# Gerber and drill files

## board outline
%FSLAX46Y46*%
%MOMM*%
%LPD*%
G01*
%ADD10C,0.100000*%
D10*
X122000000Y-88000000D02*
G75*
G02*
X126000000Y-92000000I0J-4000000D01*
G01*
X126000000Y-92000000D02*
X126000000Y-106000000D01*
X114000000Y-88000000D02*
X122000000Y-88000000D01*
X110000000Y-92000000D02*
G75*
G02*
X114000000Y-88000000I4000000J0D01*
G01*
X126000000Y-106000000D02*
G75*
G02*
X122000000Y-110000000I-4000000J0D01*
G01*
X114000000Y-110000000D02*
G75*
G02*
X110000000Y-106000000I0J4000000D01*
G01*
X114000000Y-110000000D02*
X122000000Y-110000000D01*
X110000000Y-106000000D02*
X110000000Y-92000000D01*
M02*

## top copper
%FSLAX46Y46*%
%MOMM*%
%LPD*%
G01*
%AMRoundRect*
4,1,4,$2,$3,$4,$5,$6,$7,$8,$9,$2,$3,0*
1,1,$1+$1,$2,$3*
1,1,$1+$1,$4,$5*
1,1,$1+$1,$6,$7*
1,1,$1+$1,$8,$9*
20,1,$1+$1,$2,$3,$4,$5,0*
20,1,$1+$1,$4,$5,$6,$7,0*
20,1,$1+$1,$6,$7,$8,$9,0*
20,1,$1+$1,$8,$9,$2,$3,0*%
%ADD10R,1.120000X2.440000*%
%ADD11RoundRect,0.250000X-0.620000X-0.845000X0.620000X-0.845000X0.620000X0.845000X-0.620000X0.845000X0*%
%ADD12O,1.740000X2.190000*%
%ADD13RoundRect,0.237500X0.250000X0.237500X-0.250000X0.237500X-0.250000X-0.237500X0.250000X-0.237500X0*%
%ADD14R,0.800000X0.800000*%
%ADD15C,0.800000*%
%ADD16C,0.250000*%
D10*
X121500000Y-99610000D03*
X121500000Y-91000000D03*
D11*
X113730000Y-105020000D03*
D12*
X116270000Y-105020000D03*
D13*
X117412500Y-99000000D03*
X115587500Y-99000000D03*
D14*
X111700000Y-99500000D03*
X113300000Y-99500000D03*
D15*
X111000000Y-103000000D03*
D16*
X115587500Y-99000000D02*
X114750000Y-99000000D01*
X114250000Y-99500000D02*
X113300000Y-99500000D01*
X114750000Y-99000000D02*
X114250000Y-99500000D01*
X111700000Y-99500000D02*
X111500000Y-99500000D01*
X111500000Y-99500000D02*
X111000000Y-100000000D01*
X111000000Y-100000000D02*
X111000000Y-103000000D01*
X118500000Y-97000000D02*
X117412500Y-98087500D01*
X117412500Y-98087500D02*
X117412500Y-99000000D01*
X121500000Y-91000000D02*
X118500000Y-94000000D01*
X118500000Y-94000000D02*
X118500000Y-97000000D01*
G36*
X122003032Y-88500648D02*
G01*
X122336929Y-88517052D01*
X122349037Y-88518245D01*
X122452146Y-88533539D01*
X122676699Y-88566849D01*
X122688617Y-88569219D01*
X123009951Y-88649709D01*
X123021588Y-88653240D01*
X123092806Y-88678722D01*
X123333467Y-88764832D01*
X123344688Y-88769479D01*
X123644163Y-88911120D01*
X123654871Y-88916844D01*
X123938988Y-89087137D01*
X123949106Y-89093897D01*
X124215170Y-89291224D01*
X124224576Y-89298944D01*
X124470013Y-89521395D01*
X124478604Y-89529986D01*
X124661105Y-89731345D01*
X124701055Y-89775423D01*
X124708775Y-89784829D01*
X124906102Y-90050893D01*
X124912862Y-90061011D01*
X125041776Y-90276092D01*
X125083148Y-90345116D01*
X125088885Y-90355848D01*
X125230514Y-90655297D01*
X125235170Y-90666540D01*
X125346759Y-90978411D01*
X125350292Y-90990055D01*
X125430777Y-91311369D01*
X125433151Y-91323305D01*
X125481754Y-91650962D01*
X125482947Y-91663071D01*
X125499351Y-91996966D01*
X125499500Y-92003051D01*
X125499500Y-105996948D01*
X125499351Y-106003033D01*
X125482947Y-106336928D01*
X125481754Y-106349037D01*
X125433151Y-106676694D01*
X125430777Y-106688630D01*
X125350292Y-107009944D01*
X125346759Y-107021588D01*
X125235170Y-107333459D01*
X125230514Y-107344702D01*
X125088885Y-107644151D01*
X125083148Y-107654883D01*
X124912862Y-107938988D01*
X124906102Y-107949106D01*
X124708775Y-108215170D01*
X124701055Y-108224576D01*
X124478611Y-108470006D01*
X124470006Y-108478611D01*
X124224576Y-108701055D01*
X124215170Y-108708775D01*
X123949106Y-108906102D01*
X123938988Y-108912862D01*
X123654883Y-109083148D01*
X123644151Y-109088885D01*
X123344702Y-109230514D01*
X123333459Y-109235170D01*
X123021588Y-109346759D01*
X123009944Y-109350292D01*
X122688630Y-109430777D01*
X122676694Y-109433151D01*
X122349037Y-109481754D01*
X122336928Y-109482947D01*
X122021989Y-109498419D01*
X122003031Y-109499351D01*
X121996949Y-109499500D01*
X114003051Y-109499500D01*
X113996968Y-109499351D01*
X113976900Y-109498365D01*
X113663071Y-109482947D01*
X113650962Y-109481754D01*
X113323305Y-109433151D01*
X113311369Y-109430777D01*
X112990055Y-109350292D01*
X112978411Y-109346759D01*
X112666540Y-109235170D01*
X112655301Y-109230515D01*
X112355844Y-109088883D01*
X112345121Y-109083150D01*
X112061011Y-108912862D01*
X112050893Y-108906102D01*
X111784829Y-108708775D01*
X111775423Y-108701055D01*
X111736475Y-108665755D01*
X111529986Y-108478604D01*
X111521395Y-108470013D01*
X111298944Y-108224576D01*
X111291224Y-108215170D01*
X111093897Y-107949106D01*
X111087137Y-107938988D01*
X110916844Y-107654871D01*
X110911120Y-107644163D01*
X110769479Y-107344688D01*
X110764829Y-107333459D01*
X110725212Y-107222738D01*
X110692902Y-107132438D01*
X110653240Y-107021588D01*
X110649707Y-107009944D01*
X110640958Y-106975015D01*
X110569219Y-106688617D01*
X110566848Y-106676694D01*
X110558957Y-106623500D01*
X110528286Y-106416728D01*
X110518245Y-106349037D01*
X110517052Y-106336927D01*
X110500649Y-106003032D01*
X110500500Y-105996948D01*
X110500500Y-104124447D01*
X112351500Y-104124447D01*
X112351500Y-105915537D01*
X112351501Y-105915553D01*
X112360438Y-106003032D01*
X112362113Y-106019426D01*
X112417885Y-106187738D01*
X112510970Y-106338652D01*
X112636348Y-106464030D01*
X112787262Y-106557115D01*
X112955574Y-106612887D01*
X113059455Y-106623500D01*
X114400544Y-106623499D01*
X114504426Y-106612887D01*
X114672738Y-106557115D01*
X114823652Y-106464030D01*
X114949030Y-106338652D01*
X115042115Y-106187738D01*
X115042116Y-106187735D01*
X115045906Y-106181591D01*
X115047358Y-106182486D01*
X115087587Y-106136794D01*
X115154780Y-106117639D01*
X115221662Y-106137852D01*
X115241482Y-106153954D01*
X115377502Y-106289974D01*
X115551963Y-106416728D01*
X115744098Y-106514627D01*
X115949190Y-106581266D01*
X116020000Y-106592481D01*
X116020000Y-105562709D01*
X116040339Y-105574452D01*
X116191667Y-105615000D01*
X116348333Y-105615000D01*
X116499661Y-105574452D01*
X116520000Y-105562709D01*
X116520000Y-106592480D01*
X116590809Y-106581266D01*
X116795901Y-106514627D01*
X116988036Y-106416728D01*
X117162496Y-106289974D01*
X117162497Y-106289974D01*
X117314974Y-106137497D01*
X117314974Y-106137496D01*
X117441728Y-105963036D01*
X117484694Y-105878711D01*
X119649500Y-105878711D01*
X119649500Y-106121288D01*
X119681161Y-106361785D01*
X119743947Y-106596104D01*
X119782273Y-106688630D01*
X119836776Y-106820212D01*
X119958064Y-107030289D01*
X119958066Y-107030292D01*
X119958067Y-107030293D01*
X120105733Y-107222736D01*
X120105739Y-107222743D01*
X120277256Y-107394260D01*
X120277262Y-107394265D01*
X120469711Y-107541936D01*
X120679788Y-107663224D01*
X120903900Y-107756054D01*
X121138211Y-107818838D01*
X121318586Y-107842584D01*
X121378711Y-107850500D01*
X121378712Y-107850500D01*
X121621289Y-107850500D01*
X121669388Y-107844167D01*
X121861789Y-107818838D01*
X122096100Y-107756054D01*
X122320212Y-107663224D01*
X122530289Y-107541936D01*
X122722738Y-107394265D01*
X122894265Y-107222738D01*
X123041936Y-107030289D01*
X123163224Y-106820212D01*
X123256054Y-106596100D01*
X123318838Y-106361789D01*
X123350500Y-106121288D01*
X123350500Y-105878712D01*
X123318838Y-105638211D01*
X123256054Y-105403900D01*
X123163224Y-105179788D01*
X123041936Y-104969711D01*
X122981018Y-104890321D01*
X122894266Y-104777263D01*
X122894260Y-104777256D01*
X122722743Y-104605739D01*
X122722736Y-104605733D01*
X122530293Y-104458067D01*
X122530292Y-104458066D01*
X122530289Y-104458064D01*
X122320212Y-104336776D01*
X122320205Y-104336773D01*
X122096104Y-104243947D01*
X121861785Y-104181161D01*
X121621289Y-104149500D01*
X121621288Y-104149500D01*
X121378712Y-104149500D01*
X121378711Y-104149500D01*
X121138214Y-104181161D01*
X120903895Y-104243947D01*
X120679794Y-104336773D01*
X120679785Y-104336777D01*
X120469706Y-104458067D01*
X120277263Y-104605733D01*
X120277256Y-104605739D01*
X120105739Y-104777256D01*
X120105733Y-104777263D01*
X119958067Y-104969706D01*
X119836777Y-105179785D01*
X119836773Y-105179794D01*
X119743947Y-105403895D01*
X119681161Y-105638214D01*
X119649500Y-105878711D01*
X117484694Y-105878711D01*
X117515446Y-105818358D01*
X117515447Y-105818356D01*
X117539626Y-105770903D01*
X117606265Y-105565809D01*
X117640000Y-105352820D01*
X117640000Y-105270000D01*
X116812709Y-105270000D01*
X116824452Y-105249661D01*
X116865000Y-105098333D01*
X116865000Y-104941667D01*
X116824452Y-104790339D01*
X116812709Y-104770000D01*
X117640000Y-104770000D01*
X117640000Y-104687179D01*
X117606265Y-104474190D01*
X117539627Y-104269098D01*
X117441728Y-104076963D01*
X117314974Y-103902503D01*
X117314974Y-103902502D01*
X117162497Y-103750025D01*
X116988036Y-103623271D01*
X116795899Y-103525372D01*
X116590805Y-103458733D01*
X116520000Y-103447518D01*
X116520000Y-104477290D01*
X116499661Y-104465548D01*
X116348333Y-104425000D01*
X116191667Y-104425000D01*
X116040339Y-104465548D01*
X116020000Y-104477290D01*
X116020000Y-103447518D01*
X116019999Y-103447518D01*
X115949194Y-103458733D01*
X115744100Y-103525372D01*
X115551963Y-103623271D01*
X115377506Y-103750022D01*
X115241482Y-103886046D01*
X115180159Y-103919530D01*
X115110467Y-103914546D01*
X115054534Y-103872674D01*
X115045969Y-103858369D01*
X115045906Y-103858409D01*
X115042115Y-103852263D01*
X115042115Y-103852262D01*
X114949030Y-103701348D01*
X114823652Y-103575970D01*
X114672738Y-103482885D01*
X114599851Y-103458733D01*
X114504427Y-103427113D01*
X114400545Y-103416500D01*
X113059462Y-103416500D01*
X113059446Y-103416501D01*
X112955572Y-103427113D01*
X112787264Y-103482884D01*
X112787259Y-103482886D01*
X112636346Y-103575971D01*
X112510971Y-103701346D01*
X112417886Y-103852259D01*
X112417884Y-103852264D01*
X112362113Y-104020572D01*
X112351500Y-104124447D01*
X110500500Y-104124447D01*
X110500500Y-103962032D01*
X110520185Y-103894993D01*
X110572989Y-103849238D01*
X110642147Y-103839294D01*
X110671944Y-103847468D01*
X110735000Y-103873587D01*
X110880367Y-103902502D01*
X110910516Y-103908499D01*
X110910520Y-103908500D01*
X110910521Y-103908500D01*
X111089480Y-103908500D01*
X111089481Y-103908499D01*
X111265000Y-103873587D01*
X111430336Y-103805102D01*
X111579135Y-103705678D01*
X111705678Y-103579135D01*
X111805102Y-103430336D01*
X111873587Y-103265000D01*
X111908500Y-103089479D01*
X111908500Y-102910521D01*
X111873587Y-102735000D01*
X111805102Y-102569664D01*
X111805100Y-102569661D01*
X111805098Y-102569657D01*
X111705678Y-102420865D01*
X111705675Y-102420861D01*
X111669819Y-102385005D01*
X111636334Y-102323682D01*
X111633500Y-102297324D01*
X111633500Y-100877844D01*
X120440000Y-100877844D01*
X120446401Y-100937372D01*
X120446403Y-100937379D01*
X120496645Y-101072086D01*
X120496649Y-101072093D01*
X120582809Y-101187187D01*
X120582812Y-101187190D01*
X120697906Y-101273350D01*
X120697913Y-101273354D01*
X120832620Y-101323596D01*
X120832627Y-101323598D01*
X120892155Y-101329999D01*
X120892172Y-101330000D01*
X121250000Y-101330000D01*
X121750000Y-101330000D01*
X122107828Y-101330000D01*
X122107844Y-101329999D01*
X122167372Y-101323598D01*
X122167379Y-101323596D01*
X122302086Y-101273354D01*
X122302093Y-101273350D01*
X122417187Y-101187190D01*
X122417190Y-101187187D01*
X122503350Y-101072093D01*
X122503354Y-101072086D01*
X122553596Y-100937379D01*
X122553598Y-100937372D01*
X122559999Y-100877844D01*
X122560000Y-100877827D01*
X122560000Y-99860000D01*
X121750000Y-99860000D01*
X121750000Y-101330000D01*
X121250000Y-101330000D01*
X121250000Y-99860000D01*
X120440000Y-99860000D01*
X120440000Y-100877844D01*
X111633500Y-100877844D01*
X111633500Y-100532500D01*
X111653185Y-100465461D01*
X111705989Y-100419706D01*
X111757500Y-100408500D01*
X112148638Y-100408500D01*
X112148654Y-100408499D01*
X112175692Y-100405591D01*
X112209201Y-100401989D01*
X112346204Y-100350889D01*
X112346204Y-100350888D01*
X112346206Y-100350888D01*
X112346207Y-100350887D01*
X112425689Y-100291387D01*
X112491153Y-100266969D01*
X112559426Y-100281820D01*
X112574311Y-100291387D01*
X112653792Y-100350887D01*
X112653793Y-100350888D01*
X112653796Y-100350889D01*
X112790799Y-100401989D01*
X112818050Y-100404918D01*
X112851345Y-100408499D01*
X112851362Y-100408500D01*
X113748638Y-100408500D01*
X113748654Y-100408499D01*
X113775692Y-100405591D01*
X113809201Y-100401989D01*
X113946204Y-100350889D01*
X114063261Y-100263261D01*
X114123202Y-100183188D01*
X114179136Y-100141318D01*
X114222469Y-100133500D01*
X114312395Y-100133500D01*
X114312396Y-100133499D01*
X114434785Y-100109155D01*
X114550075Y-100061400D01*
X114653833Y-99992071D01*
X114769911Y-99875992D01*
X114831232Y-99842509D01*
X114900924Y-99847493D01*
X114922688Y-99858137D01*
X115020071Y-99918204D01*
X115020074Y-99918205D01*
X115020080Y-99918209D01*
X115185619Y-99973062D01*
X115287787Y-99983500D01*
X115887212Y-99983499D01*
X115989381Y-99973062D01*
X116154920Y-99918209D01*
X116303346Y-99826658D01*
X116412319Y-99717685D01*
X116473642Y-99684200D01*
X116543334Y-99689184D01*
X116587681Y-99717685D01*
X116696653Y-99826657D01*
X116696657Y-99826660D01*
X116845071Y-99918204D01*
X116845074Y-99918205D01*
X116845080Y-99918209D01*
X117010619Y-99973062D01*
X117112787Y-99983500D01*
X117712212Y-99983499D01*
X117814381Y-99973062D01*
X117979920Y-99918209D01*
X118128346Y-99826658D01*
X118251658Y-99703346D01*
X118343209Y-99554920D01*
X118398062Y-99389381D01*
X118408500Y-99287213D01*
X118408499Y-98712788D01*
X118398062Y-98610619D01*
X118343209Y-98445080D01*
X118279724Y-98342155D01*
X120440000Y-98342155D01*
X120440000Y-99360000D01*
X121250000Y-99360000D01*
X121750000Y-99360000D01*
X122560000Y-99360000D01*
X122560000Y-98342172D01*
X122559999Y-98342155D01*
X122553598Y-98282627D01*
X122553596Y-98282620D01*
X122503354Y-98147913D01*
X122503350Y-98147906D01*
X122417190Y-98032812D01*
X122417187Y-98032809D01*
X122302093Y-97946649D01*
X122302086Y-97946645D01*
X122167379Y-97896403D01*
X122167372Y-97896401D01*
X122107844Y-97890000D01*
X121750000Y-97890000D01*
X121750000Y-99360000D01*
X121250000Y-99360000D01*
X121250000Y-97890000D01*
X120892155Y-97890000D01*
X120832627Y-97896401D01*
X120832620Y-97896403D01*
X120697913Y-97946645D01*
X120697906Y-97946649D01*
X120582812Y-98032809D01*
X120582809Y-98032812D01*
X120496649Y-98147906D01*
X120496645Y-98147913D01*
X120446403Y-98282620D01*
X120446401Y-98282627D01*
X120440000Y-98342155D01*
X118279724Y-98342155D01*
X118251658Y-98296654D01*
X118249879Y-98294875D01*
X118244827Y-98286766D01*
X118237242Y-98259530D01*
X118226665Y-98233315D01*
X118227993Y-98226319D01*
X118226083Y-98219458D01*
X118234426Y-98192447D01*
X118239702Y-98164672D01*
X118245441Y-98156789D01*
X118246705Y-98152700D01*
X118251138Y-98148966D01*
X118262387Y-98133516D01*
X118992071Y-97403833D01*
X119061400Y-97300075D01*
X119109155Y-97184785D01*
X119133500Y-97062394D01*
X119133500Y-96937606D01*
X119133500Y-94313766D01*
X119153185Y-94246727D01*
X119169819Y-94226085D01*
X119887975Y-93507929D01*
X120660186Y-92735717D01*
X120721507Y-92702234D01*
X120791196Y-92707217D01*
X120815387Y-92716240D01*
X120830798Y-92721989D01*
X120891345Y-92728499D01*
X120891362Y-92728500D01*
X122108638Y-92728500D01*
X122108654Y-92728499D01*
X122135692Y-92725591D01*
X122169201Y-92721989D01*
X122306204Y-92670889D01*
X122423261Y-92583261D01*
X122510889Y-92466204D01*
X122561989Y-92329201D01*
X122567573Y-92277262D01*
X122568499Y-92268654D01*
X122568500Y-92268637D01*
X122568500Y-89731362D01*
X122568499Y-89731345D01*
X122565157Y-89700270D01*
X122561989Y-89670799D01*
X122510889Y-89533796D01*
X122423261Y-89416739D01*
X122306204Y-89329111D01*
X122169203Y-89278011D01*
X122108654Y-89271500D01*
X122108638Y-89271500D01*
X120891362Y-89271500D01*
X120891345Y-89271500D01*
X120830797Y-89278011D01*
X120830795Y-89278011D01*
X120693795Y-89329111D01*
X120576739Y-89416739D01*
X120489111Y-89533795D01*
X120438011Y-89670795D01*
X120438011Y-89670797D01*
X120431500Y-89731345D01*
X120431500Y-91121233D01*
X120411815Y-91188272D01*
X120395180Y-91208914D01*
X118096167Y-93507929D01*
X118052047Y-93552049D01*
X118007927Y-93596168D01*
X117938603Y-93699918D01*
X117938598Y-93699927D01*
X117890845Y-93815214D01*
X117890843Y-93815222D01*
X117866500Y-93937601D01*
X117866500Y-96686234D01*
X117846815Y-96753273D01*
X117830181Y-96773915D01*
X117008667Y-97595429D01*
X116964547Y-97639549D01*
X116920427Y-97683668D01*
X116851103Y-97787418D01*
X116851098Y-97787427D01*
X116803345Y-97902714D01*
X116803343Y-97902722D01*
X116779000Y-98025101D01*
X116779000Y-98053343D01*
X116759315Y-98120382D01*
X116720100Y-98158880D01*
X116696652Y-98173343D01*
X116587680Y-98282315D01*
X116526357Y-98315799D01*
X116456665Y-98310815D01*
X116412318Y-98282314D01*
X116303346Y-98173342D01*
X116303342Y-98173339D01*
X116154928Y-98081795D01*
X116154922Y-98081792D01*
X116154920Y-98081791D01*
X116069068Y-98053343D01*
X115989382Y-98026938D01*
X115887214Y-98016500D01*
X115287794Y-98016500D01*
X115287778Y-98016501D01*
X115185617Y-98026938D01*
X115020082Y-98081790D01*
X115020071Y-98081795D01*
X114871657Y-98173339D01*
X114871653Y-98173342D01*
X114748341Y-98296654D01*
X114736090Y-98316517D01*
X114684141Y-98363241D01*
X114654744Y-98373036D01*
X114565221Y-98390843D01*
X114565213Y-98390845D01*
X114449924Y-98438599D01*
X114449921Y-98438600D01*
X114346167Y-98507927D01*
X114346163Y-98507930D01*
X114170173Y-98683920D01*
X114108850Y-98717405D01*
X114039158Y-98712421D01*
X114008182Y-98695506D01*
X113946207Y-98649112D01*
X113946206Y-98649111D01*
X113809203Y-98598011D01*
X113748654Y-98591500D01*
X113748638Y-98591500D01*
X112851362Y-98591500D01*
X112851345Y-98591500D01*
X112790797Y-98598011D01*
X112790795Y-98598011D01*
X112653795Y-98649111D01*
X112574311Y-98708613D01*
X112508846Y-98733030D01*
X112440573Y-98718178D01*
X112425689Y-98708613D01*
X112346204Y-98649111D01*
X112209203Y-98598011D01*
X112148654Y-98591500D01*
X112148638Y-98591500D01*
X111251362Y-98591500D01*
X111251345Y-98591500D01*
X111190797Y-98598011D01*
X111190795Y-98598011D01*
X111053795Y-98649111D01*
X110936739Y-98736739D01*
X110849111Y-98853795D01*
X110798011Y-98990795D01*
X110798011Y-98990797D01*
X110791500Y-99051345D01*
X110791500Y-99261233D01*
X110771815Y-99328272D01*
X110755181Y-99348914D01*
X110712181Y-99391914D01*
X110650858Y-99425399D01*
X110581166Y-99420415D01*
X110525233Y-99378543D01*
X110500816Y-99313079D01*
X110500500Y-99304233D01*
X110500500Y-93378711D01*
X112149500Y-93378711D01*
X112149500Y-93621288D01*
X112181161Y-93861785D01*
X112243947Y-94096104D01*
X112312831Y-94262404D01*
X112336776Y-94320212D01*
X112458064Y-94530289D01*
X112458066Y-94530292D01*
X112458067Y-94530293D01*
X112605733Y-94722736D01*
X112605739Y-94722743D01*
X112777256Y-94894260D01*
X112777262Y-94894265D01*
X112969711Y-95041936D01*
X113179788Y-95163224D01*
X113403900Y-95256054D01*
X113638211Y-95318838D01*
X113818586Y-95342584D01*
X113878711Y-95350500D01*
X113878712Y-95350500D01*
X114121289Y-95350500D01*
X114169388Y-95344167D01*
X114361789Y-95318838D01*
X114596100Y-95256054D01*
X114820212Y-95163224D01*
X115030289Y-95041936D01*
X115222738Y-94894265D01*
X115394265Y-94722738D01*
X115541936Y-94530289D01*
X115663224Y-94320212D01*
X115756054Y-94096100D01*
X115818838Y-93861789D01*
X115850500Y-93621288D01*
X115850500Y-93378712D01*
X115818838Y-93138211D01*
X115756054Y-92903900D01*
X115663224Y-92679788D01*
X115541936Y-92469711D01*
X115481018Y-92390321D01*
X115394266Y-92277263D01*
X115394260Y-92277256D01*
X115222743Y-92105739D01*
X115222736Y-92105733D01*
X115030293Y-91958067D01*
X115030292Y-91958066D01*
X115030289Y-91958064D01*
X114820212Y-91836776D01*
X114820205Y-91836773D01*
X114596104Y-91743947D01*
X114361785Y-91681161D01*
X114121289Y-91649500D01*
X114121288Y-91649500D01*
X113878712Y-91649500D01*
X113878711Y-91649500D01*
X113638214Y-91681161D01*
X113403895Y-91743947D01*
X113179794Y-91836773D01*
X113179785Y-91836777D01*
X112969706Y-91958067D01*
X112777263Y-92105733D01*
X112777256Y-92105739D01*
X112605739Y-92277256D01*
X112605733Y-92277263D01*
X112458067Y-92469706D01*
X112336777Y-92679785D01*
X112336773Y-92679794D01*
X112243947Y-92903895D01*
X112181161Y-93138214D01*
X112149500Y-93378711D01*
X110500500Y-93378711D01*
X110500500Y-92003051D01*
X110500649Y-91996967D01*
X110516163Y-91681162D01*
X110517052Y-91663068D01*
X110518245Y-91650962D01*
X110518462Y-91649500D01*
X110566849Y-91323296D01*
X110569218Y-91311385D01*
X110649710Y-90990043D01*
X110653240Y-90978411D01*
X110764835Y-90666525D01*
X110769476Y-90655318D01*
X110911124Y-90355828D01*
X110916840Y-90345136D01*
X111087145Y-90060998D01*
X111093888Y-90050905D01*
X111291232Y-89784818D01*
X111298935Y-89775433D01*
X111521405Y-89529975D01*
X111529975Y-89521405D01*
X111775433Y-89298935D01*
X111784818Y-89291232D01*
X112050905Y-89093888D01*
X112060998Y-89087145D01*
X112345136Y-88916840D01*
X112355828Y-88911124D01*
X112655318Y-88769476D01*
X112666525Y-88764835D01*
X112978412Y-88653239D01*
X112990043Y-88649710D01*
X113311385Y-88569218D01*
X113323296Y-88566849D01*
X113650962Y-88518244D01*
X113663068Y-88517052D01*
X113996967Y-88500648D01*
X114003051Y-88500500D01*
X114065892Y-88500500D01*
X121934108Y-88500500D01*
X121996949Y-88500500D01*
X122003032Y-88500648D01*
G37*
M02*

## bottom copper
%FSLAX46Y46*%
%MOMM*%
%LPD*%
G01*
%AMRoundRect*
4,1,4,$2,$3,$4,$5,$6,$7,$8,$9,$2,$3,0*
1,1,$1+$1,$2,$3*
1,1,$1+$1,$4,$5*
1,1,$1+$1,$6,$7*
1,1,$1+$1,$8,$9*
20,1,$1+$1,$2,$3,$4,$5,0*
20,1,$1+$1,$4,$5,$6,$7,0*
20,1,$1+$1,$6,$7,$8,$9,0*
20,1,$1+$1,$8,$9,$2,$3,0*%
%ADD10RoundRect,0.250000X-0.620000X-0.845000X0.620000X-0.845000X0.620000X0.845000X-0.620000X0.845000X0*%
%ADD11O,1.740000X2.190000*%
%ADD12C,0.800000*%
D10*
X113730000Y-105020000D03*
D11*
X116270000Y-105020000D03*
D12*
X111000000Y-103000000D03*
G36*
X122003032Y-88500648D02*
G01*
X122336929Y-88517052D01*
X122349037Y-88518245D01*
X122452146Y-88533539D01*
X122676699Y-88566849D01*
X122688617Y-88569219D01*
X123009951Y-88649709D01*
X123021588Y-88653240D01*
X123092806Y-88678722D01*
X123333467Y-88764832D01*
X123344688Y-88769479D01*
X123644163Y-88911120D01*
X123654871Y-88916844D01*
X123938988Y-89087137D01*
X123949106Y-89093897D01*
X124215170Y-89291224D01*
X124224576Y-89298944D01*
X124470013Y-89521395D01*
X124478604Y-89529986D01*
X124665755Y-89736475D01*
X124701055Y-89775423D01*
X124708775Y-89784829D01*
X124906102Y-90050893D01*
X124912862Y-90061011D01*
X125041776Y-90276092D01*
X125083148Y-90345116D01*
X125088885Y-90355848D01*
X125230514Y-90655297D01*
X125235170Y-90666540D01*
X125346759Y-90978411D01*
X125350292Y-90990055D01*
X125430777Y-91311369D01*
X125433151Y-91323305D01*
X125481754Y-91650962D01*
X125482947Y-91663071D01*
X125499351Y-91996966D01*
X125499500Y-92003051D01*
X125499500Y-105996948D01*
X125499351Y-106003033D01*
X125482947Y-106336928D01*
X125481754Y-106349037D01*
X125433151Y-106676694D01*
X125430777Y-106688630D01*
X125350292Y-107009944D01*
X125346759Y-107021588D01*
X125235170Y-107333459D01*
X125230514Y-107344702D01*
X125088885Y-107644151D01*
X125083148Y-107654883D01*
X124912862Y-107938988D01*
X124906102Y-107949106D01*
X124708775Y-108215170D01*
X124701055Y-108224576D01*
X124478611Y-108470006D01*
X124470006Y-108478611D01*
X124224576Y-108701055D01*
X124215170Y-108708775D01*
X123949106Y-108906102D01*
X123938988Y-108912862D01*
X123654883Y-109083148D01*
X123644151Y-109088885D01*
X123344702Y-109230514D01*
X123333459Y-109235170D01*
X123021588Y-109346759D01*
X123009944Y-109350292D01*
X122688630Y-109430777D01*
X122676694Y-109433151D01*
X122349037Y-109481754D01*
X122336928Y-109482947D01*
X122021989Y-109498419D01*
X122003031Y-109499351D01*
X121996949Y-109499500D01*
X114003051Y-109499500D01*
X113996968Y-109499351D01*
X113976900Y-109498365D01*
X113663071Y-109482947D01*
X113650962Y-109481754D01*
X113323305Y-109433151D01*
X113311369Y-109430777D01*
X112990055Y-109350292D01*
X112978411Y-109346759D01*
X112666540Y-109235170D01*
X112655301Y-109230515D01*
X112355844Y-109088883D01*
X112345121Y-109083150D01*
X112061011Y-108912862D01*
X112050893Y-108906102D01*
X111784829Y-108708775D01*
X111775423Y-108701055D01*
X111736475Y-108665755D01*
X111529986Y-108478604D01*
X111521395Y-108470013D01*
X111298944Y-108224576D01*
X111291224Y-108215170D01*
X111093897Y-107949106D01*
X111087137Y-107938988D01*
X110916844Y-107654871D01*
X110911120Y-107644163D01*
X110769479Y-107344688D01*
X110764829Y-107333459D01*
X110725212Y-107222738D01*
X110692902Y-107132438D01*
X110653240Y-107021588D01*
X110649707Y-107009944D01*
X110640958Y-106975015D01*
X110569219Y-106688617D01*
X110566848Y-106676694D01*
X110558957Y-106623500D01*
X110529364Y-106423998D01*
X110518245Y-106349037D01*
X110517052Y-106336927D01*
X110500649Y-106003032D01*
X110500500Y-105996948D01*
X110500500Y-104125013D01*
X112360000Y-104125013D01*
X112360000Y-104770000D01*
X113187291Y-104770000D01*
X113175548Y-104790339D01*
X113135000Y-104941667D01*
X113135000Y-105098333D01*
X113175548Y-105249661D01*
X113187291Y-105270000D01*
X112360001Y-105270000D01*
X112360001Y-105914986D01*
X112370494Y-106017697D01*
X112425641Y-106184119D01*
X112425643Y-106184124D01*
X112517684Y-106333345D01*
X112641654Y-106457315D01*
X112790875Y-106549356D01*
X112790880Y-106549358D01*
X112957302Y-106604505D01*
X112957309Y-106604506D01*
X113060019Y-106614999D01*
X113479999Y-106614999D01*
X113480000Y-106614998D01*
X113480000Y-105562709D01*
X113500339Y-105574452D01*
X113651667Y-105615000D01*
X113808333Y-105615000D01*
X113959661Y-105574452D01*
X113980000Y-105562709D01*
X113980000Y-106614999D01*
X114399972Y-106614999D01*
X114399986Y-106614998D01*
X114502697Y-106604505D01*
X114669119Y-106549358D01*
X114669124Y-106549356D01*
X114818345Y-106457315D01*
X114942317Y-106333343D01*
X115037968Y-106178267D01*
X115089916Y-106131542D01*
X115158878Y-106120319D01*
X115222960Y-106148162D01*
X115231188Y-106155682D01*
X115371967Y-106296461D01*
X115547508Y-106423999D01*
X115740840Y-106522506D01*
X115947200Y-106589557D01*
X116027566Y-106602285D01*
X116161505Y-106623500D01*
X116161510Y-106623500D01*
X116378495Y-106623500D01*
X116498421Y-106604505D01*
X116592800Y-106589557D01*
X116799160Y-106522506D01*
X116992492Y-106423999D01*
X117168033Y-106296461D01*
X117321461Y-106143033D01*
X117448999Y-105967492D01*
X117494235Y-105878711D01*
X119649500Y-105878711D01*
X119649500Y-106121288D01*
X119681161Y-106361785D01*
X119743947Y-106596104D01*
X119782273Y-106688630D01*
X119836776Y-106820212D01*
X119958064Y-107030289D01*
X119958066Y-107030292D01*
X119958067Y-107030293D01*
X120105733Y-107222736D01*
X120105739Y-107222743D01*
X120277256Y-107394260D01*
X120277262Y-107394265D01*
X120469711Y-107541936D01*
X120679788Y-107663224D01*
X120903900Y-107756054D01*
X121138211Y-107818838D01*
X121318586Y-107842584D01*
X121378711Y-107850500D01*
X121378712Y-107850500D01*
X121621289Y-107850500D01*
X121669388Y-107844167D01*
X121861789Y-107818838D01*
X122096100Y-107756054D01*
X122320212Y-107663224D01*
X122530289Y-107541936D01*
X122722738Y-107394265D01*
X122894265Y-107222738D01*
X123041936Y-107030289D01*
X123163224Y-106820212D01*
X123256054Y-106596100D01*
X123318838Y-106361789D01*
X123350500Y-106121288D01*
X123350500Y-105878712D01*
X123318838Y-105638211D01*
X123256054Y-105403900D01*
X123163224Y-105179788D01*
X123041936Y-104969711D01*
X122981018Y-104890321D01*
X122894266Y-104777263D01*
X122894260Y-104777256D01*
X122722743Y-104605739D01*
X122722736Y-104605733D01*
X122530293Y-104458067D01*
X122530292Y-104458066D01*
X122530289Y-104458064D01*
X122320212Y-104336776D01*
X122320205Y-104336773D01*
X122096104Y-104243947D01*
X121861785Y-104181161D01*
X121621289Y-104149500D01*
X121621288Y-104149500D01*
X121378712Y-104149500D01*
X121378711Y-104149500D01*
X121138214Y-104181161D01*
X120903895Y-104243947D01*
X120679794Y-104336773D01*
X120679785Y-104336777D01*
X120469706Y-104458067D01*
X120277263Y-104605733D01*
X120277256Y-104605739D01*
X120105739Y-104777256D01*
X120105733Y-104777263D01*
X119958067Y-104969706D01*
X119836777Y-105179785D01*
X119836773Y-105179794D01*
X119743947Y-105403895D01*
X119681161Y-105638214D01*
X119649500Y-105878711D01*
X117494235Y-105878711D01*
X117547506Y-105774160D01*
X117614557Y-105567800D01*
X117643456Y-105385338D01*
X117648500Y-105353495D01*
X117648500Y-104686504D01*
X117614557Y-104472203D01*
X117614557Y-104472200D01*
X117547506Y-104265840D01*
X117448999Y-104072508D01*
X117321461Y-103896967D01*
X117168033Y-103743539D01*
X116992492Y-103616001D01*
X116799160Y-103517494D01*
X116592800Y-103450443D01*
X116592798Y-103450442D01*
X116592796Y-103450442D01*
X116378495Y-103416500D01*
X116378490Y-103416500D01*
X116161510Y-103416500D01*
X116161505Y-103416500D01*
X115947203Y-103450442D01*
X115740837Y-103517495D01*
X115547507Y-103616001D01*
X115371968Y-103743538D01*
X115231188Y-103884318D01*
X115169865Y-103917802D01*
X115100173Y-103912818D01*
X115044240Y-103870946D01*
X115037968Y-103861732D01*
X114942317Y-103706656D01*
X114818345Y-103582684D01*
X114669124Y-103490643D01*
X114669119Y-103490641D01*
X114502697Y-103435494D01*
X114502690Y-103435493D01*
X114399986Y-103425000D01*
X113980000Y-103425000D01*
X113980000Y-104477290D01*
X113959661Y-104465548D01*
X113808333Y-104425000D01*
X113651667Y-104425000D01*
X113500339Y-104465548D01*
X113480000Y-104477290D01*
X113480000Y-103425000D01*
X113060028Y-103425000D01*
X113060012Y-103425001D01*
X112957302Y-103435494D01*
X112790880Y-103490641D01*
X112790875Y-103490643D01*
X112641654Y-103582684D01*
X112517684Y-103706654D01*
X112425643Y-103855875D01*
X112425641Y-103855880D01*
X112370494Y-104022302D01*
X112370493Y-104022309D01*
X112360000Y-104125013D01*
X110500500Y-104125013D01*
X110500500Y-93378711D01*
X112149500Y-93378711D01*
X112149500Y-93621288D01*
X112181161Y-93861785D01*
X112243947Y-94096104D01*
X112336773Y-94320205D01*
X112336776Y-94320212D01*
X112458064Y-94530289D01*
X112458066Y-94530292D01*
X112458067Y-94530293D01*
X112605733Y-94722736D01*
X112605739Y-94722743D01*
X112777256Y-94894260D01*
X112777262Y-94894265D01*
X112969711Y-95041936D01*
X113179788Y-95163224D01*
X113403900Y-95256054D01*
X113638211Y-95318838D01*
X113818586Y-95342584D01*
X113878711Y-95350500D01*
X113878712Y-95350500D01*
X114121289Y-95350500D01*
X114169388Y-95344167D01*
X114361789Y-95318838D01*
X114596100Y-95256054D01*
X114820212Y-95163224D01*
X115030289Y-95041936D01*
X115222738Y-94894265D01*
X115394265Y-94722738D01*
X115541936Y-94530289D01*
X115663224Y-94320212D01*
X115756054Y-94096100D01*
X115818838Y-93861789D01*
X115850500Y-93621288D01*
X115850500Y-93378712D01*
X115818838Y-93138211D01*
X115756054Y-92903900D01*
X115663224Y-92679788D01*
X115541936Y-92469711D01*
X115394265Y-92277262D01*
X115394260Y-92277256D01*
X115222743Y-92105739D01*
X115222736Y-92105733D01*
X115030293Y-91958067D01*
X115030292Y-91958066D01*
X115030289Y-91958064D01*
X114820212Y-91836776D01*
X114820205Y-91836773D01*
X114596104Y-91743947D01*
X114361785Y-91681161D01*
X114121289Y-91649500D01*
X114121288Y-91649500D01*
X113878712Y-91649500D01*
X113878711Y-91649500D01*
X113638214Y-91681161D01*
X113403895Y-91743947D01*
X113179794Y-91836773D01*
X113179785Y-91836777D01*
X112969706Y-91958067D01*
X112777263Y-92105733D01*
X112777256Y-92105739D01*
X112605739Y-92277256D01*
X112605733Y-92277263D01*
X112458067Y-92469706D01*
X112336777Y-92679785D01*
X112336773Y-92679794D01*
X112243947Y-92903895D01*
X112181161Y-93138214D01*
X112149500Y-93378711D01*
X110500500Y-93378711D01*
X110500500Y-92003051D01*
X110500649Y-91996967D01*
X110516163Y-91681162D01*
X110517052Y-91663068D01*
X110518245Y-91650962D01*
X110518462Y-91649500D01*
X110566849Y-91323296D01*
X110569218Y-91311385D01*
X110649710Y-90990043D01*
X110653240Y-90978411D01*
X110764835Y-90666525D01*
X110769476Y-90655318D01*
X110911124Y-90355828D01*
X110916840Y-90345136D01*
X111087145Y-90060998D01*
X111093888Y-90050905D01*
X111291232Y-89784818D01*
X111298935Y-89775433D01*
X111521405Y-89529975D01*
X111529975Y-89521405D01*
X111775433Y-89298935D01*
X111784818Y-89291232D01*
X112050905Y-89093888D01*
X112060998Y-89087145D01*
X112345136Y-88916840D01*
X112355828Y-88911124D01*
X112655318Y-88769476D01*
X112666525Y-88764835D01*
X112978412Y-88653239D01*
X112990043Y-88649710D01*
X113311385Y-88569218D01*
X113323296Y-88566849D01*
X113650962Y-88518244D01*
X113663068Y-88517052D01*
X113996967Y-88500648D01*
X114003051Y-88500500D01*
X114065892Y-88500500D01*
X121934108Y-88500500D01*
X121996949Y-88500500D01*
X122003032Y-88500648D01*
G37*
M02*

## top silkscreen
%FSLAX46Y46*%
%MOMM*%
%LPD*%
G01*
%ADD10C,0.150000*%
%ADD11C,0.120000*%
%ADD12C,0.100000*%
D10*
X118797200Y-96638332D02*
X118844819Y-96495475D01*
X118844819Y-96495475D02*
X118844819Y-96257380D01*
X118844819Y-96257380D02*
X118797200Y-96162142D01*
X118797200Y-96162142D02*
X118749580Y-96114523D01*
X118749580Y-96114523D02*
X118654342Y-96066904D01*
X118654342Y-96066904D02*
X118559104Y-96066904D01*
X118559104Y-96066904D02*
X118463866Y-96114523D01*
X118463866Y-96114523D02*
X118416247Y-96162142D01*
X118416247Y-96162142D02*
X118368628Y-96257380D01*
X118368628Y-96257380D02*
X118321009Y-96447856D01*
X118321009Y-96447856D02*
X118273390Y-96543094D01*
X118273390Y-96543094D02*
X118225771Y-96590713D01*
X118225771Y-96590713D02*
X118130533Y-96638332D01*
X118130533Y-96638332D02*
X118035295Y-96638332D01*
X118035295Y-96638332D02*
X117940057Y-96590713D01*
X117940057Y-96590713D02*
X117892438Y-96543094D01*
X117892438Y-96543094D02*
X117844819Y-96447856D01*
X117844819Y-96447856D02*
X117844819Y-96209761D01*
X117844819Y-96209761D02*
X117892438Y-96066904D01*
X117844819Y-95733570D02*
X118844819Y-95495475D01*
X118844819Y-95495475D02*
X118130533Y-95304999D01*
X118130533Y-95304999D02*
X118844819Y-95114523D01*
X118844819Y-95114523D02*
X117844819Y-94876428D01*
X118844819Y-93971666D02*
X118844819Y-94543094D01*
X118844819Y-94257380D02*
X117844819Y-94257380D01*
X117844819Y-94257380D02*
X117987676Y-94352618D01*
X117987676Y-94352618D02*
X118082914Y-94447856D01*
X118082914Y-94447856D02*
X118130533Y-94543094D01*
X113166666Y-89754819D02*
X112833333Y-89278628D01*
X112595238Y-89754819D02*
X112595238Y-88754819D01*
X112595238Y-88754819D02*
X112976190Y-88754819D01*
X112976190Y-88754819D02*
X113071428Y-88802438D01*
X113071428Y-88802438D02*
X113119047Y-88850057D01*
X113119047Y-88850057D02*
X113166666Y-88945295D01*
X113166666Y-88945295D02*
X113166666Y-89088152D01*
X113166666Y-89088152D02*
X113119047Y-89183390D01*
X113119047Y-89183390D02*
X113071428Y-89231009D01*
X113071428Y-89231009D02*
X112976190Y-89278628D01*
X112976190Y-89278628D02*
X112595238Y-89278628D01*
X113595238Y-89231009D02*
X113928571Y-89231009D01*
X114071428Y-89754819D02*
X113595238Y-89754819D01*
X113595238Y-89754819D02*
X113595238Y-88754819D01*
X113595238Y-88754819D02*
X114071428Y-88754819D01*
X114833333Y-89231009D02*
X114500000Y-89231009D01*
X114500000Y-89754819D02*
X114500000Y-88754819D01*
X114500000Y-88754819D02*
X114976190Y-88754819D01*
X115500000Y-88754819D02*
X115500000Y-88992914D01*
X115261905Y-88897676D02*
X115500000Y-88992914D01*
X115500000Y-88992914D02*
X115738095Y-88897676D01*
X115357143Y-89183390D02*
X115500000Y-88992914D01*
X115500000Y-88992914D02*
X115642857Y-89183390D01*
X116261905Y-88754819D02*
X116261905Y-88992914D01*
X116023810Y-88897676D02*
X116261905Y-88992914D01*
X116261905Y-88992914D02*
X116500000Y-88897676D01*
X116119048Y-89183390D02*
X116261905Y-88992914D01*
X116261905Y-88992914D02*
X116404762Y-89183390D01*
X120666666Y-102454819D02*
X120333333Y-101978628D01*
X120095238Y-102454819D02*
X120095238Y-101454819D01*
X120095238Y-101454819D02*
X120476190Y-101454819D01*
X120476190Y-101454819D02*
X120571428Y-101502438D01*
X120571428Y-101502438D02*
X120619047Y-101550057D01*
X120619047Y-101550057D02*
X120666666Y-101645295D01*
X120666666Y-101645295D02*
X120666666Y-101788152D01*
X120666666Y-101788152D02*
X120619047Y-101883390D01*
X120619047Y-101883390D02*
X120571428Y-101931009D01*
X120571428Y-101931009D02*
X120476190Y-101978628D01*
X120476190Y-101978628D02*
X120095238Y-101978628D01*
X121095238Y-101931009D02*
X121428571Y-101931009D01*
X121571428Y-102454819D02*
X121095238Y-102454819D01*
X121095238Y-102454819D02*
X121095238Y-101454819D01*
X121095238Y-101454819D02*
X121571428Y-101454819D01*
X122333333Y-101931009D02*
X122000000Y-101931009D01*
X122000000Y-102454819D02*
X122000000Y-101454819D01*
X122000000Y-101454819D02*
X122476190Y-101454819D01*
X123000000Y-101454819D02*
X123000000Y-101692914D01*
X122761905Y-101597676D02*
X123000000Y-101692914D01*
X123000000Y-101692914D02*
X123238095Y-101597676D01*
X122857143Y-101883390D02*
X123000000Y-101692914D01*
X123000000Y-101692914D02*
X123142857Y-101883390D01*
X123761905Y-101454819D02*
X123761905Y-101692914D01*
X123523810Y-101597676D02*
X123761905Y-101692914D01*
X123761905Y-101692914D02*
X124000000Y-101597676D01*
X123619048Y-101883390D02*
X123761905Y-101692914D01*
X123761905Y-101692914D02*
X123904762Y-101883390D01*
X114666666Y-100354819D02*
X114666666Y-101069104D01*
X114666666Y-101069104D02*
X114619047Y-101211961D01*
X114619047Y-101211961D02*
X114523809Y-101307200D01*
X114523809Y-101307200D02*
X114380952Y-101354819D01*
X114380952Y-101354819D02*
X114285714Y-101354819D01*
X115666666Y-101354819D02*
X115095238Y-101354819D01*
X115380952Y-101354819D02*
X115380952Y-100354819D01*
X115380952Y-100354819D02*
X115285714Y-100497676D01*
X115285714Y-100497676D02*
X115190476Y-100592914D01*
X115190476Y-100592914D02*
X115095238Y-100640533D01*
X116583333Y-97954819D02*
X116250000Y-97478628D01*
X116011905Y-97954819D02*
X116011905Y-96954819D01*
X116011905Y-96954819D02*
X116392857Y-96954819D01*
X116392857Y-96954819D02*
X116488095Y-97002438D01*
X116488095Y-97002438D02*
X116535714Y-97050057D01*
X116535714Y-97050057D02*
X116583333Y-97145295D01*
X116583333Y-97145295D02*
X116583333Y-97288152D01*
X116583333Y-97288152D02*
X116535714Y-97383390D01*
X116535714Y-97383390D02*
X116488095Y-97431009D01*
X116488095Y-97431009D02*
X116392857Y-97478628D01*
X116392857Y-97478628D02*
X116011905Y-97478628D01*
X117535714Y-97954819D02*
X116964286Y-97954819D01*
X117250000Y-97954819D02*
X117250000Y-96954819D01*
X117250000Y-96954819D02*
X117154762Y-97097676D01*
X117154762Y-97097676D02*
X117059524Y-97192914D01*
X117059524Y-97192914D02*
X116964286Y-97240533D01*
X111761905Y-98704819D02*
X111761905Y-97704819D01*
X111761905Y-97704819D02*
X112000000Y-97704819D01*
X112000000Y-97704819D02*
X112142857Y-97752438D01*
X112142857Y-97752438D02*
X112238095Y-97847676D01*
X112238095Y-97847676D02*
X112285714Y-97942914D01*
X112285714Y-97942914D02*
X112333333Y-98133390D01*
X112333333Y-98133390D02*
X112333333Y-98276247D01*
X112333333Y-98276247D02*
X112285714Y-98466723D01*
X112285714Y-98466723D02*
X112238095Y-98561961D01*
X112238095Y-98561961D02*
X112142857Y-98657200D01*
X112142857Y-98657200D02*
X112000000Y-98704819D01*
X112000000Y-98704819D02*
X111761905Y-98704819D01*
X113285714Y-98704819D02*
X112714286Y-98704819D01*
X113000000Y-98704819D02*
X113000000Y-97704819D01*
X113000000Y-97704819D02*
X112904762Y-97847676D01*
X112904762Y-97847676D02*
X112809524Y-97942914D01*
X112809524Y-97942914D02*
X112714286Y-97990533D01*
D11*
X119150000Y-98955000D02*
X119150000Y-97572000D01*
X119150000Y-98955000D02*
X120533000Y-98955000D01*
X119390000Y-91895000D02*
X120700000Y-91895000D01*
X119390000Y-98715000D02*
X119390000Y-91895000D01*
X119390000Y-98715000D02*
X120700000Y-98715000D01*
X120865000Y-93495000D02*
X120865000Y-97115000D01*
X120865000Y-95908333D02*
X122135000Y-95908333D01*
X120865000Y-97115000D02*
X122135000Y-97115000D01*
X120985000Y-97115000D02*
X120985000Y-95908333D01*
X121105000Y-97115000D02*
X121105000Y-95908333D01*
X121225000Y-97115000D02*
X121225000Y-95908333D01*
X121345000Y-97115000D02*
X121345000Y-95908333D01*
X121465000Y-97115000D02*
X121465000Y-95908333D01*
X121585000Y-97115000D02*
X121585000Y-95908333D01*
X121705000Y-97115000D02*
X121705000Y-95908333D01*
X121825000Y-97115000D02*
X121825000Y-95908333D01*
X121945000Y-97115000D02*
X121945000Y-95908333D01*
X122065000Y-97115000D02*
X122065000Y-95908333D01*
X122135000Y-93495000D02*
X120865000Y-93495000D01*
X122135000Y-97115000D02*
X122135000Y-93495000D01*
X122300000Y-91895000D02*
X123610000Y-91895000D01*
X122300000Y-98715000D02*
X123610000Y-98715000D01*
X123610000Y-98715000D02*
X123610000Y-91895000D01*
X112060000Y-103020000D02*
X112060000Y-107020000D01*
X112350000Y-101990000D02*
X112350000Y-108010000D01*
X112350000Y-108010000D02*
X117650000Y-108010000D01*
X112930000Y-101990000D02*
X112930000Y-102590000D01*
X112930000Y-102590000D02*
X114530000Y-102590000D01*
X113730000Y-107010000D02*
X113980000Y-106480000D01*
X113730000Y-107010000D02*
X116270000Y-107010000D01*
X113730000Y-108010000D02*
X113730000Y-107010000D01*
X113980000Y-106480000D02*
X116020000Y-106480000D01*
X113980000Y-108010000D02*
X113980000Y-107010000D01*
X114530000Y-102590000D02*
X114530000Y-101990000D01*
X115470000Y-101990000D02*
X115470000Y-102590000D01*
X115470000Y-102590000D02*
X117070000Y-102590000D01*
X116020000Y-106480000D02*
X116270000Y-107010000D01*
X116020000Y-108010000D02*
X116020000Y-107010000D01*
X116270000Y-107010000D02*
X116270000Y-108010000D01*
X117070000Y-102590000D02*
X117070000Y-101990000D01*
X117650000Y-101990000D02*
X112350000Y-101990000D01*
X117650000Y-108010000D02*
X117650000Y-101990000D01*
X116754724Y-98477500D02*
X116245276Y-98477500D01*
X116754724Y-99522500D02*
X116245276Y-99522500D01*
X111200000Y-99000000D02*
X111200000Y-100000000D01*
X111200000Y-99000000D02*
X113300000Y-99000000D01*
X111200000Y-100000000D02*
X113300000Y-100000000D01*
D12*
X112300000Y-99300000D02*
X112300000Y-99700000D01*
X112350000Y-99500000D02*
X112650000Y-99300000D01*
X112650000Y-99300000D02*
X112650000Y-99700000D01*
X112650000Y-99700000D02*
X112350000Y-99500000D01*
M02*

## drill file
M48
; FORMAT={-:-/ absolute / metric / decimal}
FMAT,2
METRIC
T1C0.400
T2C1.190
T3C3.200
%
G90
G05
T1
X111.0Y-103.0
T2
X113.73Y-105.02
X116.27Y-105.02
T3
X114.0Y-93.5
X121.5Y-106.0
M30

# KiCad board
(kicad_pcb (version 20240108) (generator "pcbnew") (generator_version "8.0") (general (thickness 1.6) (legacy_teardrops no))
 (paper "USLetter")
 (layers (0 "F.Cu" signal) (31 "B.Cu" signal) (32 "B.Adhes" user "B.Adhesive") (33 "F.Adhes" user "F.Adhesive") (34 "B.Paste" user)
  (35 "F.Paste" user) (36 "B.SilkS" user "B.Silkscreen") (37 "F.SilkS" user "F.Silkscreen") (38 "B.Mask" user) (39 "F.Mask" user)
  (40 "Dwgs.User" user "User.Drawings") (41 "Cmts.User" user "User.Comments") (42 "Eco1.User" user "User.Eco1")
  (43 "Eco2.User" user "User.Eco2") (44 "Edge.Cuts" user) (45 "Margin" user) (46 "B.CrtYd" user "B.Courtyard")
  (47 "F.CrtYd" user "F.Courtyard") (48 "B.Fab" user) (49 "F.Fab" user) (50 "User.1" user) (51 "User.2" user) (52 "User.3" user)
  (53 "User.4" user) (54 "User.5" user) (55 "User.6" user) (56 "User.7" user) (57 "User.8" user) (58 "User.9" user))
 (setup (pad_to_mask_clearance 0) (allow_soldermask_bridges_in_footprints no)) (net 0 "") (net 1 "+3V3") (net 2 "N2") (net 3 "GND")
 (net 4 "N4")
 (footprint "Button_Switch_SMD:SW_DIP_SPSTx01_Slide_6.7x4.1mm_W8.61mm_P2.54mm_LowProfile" (layer "F.Cu") (at 121.5 95.305 90)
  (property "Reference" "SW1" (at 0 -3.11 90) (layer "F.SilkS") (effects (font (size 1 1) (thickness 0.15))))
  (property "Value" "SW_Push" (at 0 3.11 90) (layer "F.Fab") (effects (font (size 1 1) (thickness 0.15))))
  (fp_line (start -3.65 -2.35) (end -2.267 -2.35) (stroke (width 0.12) (type solid)) (layer "F.SilkS"))
  (fp_line (start -3.65 -2.35) (end -3.65 -0.967) (stroke (width 0.12) (type solid)) (layer "F.SilkS"))
  (fp_line (start 3.41 -2.11) (end 3.41 -0.8) (stroke (width 0.12) (type solid)) (layer "F.SilkS"))
  (fp_line (start -3.41 -2.11) (end 3.41 -2.11) (stroke (width 0.12) (type solid)) (layer "F.SilkS"))
  (fp_line (start -3.41 -2.11) (end -3.41 -0.8) (stroke (width 0.12) (type solid)) (layer "F.SilkS"))
  (fp_line (start 1.81 -0.635) (end -1.81 -0.635) (stroke (width 0.12) (type solid)) (layer "F.SilkS"))
  (fp_line (start -0.603333 -0.635) (end -0.603333 0.635) (stroke (width 0.12) (type solid)) (layer "F.SilkS"))
  (fp_line (start -1.81 -0.635) (end -1.81 0.635) (stroke (width 0.12) (type solid)) (layer "F.SilkS"))
  (fp_line (start -1.81 -0.515) (end -0.603333 -0.515) (stroke (width 0.12) (type solid)) (layer "F.SilkS"))
  (fp_line (start -1.81 -0.395) (end -0.603333 -0.395) (stroke (width 0.12) (type solid)) (layer "F.SilkS"))
  (fp_line (start -1.81 -0.275) (end -0.603333 -0.275) (stroke (width 0.12) (type solid)) (layer "F.SilkS"))
  (fp_line (start -1.81 -0.155) (end -0.603333 -0.155) (stroke (width 0.12) (type solid)) (layer "F.SilkS"))
  (fp_line (start -1.81 -0.035) (end -0.603333 -0.035) (stroke (width 0.12) (type solid)) (layer "F.SilkS"))
  (fp_line (start -1.81 0.085) (end -0.603333 0.085) (stroke (width 0.12) (type solid)) (layer "F.SilkS"))
  (fp_line (start -1.81 0.205) (end -0.603333 0.205) (stroke (width 0.12) (type solid)) (layer "F.SilkS"))
  (fp_line (start -1.81 0.325) (end -0.603333 0.325) (stroke (width 0.12) (type solid)) (layer "F.SilkS"))
  (fp_line (start -1.81 0.445) (end -0.603333 0.445) (stroke (width 0.12) (type solid)) (layer "F.SilkS"))
  (fp_line (start -1.81 0.565) (end -0.603333 0.565) (stroke (width 0.12) (type solid)) (layer "F.SilkS"))
  (fp_line (start 1.81 0.635) (end 1.81 -0.635) (stroke (width 0.12) (type solid)) (layer "F.SilkS"))
  (fp_line (start -1.81 0.635) (end 1.81 0.635) (stroke (width 0.12) (type solid)) (layer "F.SilkS"))
  (fp_line (start 3.41 0.8) (end 3.41 2.11) (stroke (width 0.12) (type solid)) (layer "F.SilkS"))
  (fp_line (start -3.41 0.8) (end -3.41 2.11) (stroke (width 0.12) (type solid)) (layer "F.SilkS"))
  (fp_line (start -3.41 2.11) (end 3.41 2.11) (stroke (width 0.12) (type solid)) (layer "F.SilkS"))
  (pad "1" smd rect (at -4.305 0 90) (size 2.44 1.12) (layers "F.Cu" "F.Paste" "F.Mask") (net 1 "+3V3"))
  (pad "2" smd rect (at 4.305 0 90) (size 2.44 1.12) (layers "F.Cu" "F.Paste" "F.Mask") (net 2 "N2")))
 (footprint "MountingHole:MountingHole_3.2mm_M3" (layer "F.Cu") (at 114 93.5)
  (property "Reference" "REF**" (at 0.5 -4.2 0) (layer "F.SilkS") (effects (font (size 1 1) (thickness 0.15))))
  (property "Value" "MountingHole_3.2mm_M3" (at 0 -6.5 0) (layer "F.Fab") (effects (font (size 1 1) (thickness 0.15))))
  (pad "" np_thru_hole circle (at 0 0) (size 3.2 3.2) (drill 3.2) (layers "*.Cu" "*.Mask")))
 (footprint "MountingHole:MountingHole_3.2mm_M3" (layer "F.Cu") (at 121.5 106)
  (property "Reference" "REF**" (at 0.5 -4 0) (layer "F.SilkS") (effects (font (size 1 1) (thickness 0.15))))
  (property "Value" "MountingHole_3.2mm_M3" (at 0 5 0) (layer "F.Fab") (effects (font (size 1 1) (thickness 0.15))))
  (pad "" np_thru_hole circle (at 0 0) (size 3.2 3.2) (drill 3.2) (layers "*.Cu" "*.Mask")))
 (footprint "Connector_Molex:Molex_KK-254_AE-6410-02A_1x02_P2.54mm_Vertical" (layer "F.Cu") (at 113.73 105.02)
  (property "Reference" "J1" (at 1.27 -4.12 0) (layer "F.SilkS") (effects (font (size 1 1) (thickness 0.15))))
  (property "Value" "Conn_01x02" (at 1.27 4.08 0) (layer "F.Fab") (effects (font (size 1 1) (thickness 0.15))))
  (fp_line (start -1.67 -2) (end -1.67 2) (stroke (width 0.12) (type solid)) (layer "F.SilkS"))
  (fp_line (start -1.38 -3.03) (end -1.38 2.99) (stroke (width 0.12) (type solid)) (layer "F.SilkS"))
  (fp_line (start -1.38 2.99) (end 3.92 2.99) (stroke (width 0.12) (type solid)) (layer "F.SilkS"))
  (fp_line (start -0.8 -3.03) (end -0.8 -2.43) (stroke (width 0.12) (type solid)) (layer "F.SilkS"))
  (fp_line (start -0.8 -2.43) (end 0.8 -2.43) (stroke (width 0.12) (type solid)) (layer "F.SilkS"))
  (fp_line (start 0 1.99) (end 0.25 1.46) (stroke (width 0.12) (type solid)) (layer "F.SilkS"))
  (fp_line (start 0 1.99) (end 2.54 1.99) (stroke (width 0.12) (type solid)) (layer "F.SilkS"))
  (fp_line (start 0 2.99) (end 0 1.99) (stroke (width 0.12) (type solid)) (layer "F.SilkS"))
  (fp_line (start 0.25 1.46) (end 2.29 1.46) (stroke (width 0.12) (type solid)) (layer "F.SilkS"))
  (fp_line (start 0.25 2.99) (end 0.25 1.99) (stroke (width 0.12) (type solid)) (layer "F.SilkS"))
  (fp_line (start 0.8 -2.43) (end 0.8 -3.03) (stroke (width 0.12) (type solid)) (layer "F.SilkS"))
  (fp_line (start 1.74 -3.03) (end 1.74 -2.43) (stroke (width 0.12) (type solid)) (layer "F.SilkS"))
  (fp_line (start 1.74 -2.43) (end 3.34 -2.43) (stroke (width 0.12) (type solid)) (layer "F.SilkS"))
  (fp_line (start 2.29 1.46) (end 2.54 1.99) (stroke (width 0.12) (type solid)) (layer "F.SilkS"))
  (fp_line (start 2.29 2.99) (end 2.29 1.99) (stroke (width 0.12) (type solid)) (layer "F.SilkS"))
  (fp_line (start 2.54 1.99) (end 2.54 2.99) (stroke (width 0.12) (type solid)) (layer "F.SilkS"))
  (fp_line (start 3.34 -2.43) (end 3.34 -3.03) (stroke (width 0.12) (type solid)) (layer "F.SilkS"))
  (fp_line (start 3.92 -3.03) (end -1.38 -3.03) (stroke (width 0.12) (type solid)) (layer "F.SilkS"))
  (fp_line (start 3.92 2.99) (end 3.92 -3.03) (stroke (width 0.12) (type solid)) (layer "F.SilkS"))
  (pad "1" thru_hole roundrect (at 0 0) (size 1.74 2.19) (drill 1.19) (layers "*.Cu" "*.Mask") (remove_unused_layers no)
   (roundrect_rratio 0.143678) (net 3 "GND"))
  (pad "2" thru_hole oval (at 2.54 0) (size 1.74 2.19) (drill 1.19) (layers "*.Cu" "*.Mask") (remove_unused_layers no) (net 1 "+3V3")))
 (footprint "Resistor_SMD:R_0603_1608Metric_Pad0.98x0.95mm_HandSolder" (layer "F.Cu") (at 116.5 99 180)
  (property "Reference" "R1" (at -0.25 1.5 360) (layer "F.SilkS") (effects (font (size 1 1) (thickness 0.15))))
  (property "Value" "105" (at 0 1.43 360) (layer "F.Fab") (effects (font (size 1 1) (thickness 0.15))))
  (fp_line (start -0.254724 0.5225) (end 0.254724 0.5225) (stroke (width 0.12) (type solid)) (layer "F.SilkS"))
  (fp_line (start -0.254724 -0.5225) (end 0.254724 -0.5225) (stroke (width 0.12) (type solid)) (layer "F.SilkS"))
  (pad "1" smd roundrect (at -0.9125 0 180) (size 0.975 0.95) (layers "F.Cu" "F.Paste" "F.Mask") (roundrect_rratio 0.25) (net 2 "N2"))
  (pad "2" smd roundrect (at 0.9125 0 180) (size 0.975 0.95) (layers "F.Cu" "F.Paste" "F.Mask") (roundrect_rratio 0.25) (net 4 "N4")))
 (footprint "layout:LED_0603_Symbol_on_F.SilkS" (layer "F.Cu") (at 112.5 99.5)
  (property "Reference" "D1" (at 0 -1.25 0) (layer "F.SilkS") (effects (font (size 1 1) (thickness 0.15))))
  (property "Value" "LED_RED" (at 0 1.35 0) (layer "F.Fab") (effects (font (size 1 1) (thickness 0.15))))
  (fp_line (start -1.3 -0.5) (end -1.3 0.5) (stroke (width 0.12) (type solid)) (layer "F.SilkS"))
  (fp_line (start -1.3 -0.5) (end 0.8 -0.5) (stroke (width 0.12) (type solid)) (layer "F.SilkS"))
  (fp_line (start -1.3 0.5) (end 0.8 0.5) (stroke (width 0.12) (type solid)) (layer "F.SilkS"))
  (fp_line (start -0.2 -0.2) (end -0.2 0.2) (stroke (width 0.1) (type solid)) (layer "F.SilkS"))
  (fp_line (start -0.15 0) (end 0.15 -0.2) (stroke (width 0.1) (type solid)) (layer "F.SilkS"))
  (fp_line (start 0.15 -0.2) (end 0.15 0.2) (stroke (width 0.1) (type solid)) (layer "F.SilkS"))
  (fp_line (start 0.15 0.2) (end -0.15 0) (stroke (width 0.1) (type solid)) (layer "F.SilkS"))
  (pad "1" smd rect (at -0.8 0 180) (size 0.8 0.8) (layers "F.Cu" "F.Paste" "F.Mask") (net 3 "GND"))
  (pad "2" smd rect (at 0.8 0 180) (size 0.8 0.8) (layers "F.Cu" "F.Paste" "F.Mask") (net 4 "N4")))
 (gr_arc (start 122 88) (mid 124.828427 89.171573) (end 126 92) (stroke (width 0.1) (type default)) (layer "Edge.Cuts"))
 (gr_line (start 126 92) (end 126 106) (stroke (width 0.1) (type default)) (layer "Edge.Cuts"))
 (gr_line (start 114 88) (end 122 88) (stroke (width 0.1) (type default)) (layer "Edge.Cuts"))
 (gr_arc (start 110 92) (mid 111.171573 89.171573) (end 114 88) (stroke (width 0.1) (type default)) (layer "Edge.Cuts"))
 (gr_arc (start 126 106) (mid 124.828427 108.828427) (end 122 110) (stroke (width 0.1) (type default)) (layer "Edge.Cuts"))
 (gr_arc (start 114 110) (mid 111.171573 108.828427) (end 110 106) (stroke (width 0.1) (type default)) (layer "Edge.Cuts"))
 (gr_line (start 114 110) (end 122 110) (stroke (width 0.1) (type default)) (layer "Edge.Cuts"))
 (gr_line (start 110 106) (end 110 92) (stroke (width 0.1) (type default)) (layer "Edge.Cuts"))
 (segment (start 115.5875 99) (end 114.75 99) (width 0.25) (layer "F.Cu") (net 4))
 (segment (start 114.25 99.5) (end 113.3 99.5) (width 0.25) (layer "F.Cu") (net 4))
 (segment (start 114.75 99) (end 114.25 99.5) (width 0.25) (layer "F.Cu") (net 4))
 (segment (start 111.7 99.5) (end 111.5 99.5) (width 0.25) (layer "F.Cu") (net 3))
 (segment (start 111.5 99.5) (end 111 100) (width 0.25) (layer "F.Cu") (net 3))
 (segment (start 111 100) (end 111 103) (width 0.25) (layer "F.Cu") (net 3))
 (via (at 111 103) (size 0.8) (drill 0.4) (layers "F.Cu" "B.Cu") (free yes) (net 3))
 (segment (start 118.5 97) (end 117.4125 98.0875) (width 0.25) (layer "F.Cu") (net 2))
 (segment (start 117.4125 98.0875) (end 117.4125 99) (width 0.25) (layer "F.Cu") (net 2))
 (segment (start 121.5 91) (end 118.5 94) (width 0.25) (layer "F.Cu") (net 2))
 (segment (start 118.5 94) (end 118.5 97) (width 0.25) (layer "F.Cu") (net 2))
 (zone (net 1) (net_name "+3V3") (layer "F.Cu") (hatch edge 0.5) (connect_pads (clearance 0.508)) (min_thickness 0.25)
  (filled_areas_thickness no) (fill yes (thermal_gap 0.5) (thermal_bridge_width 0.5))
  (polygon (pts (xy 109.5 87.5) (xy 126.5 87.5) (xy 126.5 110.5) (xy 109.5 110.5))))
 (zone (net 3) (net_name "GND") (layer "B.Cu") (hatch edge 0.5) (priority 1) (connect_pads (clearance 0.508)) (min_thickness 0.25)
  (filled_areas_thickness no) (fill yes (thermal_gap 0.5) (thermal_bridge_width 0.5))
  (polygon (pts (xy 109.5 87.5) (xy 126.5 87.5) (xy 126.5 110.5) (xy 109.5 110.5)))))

